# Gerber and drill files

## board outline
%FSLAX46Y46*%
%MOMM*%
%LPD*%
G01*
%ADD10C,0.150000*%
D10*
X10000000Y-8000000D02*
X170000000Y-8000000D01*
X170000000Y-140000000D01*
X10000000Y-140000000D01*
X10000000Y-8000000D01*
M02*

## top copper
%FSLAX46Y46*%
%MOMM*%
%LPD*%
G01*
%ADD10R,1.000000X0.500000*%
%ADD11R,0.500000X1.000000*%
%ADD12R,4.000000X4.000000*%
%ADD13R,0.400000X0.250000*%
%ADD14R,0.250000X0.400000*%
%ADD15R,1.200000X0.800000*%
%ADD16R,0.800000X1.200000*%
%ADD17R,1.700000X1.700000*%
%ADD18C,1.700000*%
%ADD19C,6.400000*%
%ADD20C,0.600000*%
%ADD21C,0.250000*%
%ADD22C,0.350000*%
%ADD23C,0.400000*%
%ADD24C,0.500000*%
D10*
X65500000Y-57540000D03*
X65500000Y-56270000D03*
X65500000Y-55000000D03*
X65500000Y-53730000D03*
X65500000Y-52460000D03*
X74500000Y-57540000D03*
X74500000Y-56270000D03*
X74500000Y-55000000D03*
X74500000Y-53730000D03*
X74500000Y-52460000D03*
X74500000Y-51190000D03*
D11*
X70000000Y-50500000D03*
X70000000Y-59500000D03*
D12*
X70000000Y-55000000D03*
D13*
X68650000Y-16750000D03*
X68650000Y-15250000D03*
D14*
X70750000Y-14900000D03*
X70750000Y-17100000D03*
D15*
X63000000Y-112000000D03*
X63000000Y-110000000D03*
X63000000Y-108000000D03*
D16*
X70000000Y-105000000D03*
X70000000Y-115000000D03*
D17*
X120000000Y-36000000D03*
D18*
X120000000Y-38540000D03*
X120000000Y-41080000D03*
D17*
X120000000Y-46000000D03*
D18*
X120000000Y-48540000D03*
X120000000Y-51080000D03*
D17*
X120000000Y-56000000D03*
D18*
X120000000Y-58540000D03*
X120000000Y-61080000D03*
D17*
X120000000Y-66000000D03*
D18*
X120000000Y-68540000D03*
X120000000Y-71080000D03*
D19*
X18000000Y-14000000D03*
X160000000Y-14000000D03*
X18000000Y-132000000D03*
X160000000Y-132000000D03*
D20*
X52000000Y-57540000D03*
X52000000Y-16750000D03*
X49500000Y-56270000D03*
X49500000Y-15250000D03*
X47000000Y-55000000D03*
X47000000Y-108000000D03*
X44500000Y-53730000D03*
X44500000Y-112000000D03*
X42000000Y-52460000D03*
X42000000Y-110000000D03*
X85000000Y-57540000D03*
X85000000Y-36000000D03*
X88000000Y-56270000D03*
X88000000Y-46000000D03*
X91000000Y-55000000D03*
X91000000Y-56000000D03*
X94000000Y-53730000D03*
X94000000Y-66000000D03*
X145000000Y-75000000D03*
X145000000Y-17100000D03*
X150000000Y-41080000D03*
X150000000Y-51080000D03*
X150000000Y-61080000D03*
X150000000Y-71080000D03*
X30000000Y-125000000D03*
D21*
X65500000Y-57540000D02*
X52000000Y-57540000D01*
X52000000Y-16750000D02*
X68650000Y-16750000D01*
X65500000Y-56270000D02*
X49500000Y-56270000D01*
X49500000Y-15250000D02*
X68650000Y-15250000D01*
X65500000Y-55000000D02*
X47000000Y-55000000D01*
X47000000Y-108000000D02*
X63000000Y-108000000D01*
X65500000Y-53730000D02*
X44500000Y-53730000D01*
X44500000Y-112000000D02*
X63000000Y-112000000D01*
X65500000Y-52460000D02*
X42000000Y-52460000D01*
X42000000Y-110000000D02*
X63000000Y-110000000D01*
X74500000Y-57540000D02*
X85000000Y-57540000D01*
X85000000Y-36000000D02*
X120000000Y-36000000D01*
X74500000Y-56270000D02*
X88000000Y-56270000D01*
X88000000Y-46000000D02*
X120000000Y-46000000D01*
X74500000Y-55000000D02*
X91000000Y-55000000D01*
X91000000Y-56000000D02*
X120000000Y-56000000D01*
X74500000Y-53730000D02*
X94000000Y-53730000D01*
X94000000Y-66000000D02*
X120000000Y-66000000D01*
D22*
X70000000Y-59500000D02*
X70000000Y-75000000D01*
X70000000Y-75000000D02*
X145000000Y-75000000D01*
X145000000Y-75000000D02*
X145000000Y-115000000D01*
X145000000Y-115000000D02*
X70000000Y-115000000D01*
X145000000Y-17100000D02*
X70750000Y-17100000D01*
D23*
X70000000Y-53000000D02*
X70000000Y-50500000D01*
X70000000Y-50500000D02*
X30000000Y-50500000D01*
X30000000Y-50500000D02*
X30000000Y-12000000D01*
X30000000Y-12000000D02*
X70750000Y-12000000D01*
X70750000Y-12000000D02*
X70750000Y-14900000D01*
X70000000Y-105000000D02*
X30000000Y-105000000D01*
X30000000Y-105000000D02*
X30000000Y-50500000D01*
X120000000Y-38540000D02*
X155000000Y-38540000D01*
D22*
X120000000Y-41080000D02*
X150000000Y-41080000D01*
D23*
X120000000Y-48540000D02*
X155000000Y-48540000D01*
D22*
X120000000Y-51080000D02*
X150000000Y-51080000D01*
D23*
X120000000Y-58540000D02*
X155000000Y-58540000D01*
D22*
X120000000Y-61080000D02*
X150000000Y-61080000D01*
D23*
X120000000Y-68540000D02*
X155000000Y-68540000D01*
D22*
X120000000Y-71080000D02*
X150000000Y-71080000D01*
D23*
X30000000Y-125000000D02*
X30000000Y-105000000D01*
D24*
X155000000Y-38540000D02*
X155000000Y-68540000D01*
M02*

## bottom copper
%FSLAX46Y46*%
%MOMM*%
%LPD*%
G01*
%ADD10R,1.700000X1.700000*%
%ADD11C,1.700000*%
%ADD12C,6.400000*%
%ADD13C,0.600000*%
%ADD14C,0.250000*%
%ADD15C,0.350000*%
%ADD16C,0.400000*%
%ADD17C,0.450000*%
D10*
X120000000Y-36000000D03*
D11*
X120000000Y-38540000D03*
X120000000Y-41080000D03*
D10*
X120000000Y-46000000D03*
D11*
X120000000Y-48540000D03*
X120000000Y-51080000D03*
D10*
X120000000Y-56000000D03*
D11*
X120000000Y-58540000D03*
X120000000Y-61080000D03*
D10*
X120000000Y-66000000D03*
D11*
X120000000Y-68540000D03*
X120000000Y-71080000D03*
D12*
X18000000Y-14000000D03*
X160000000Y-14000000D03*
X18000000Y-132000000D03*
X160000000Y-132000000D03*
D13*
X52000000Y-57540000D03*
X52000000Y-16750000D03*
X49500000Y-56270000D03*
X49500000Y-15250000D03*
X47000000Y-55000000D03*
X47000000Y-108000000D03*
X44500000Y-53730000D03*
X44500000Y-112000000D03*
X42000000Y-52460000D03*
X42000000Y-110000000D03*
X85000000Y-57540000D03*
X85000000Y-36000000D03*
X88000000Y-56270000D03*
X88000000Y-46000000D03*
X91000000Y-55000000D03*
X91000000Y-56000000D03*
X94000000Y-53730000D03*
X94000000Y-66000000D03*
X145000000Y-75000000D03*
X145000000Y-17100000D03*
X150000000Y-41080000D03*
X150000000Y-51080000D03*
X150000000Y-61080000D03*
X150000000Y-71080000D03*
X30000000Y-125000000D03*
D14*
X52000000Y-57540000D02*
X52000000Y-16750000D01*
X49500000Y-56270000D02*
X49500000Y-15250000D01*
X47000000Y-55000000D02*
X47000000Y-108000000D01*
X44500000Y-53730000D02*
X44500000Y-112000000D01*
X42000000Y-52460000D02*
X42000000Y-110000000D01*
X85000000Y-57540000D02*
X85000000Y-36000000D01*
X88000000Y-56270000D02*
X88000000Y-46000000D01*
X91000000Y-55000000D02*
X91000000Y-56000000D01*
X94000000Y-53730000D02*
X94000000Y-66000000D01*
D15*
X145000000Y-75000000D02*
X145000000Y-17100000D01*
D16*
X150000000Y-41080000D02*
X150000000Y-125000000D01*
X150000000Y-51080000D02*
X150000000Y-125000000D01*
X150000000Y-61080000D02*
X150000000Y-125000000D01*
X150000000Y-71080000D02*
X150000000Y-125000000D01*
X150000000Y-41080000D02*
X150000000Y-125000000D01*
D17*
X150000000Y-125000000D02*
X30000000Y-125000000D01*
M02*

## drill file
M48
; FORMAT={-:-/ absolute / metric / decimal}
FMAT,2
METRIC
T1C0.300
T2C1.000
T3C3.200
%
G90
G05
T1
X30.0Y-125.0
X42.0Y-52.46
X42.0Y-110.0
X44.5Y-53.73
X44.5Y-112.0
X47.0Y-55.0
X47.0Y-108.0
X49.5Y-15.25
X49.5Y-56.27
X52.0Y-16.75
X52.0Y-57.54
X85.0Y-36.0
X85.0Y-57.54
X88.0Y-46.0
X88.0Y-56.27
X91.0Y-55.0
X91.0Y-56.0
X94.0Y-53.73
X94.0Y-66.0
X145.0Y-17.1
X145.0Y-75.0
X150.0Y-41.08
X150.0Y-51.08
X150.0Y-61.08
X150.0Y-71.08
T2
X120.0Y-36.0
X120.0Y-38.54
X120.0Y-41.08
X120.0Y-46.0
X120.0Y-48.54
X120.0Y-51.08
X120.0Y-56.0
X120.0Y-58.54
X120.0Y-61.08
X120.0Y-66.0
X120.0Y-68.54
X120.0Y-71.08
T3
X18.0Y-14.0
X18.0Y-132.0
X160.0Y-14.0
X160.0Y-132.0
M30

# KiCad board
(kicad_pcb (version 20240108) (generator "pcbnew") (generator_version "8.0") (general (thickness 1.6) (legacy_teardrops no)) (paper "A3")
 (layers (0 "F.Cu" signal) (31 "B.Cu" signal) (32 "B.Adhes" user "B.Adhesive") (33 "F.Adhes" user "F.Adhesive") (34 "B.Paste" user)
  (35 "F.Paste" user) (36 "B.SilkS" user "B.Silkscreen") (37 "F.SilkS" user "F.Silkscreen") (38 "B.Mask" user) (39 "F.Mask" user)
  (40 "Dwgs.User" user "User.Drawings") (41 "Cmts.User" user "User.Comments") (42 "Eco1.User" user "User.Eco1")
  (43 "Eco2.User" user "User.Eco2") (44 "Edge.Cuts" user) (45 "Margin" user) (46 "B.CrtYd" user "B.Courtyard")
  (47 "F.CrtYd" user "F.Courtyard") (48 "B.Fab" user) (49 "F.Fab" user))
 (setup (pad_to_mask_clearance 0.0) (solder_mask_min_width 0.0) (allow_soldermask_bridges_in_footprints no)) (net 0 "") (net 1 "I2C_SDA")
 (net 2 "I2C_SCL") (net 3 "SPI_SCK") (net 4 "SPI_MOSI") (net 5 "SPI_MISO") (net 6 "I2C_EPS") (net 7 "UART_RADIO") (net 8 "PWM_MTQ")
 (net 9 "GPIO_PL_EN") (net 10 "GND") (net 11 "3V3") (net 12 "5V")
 (gr_rect (start 10 8) (end 170 140) (stroke (width 0.15) (type solid)) (fill none) (layer "Edge.Cuts"))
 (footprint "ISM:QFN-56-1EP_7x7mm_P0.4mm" (layer "F.Cu") (at 70 55)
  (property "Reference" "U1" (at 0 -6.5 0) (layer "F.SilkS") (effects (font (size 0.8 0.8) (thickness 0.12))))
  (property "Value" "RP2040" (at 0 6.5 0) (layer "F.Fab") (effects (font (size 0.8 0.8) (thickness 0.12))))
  (pad "1" smd rect (at -4.5 2.54) (size 1.0 0.5) (layers "F.Cu" "F.Paste" "F.Mask") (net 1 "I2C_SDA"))
  (pad "2" smd rect (at -4.5 1.27) (size 1.0 0.5) (layers "F.Cu" "F.Paste" "F.Mask") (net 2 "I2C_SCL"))
  (pad "3" smd rect (at -4.5 0) (size 1.0 0.5) (layers "F.Cu" "F.Paste" "F.Mask") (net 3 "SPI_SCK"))
  (pad "4" smd rect (at -4.5 -1.27) (size 1.0 0.5) (layers "F.Cu" "F.Paste" "F.Mask") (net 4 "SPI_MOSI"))
  (pad "5" smd rect (at -4.5 -2.54) (size 1.0 0.5) (layers "F.Cu" "F.Paste" "F.Mask") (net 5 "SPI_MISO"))
  (pad "6" smd rect (at 4.5 2.54) (size 1.0 0.5) (layers "F.Cu" "F.Paste" "F.Mask") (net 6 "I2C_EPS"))
  (pad "7" smd rect (at 4.5 1.27) (size 1.0 0.5) (layers "F.Cu" "F.Paste" "F.Mask") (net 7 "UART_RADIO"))
  (pad "8" smd rect (at 4.5 0) (size 1.0 0.5) (layers "F.Cu" "F.Paste" "F.Mask") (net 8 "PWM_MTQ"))
  (pad "9" smd rect (at 4.5 -1.27) (size 1.0 0.5) (layers "F.Cu" "F.Paste" "F.Mask") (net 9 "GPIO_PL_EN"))
  (pad "12" smd rect (at 4.5 -2.54) (size 1.0 0.5) (layers "F.Cu" "F.Paste" "F.Mask"))
  (pad "13" smd rect (at 4.5 -3.81) (size 1.0 0.5) (layers "F.Cu" "F.Paste" "F.Mask"))
  (pad "10" smd rect (at 0 -4.5) (size 0.5 1.0) (layers "F.Cu" "F.Paste" "F.Mask") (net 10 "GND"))
  (pad "11" smd rect (at 0 4.5) (size 0.5 1.0) (layers "F.Cu" "F.Paste" "F.Mask") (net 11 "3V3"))
  (pad "EP" smd rect (at 0 0) (size 4 4) (layers "F.Cu" "F.Paste" "F.Mask") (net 10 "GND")))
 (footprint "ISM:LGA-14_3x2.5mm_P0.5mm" (layer "F.Cu") (at 70 16)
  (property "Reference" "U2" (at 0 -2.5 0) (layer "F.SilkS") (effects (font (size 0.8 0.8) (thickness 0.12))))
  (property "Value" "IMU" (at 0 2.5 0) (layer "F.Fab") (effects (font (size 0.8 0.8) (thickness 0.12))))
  (pad "1" smd rect (at -1.35 0.75) (size 0.4 0.25) (layers "F.Cu" "F.Paste" "F.Mask") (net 1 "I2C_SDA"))
  (pad "2" smd rect (at -1.35 -0.75) (size 0.4 0.25) (layers "F.Cu" "F.Paste" "F.Mask") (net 2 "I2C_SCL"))
  (pad "3" smd rect (at 0.75 -1.1) (size 0.25 0.4) (layers "F.Cu" "F.Paste" "F.Mask") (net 10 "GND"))
  (pad "4" smd rect (at 0.75 1.1) (size 0.25 0.4) (layers "F.Cu" "F.Paste" "F.Mask") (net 11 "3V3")))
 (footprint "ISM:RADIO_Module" (layer "F.Cu") (at 70 110)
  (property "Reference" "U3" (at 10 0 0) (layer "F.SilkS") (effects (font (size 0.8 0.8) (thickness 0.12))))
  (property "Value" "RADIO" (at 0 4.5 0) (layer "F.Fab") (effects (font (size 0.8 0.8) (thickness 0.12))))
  (pad "1" smd rect (at -7 2) (size 1.2 0.8) (layers "F.Cu" "F.Paste" "F.Mask") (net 4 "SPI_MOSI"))
  (pad "2" smd rect (at -7 0) (size 1.2 0.8) (layers "F.Cu" "F.Paste" "F.Mask") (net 5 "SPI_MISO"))
  (pad "3" smd rect (at -7 -2) (size 1.2 0.8) (layers "F.Cu" "F.Paste" "F.Mask") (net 3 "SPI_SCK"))
  (pad "4" smd rect (at 0 -5) (size 0.8 1.2) (layers "F.Cu" "F.Paste" "F.Mask") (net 10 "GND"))
  (pad "5" smd rect (at 0 5) (size 0.8 1.2) (layers "F.Cu" "F.Paste" "F.Mask") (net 11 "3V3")))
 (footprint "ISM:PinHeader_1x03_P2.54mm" (layer "F.Cu") (at 120 36)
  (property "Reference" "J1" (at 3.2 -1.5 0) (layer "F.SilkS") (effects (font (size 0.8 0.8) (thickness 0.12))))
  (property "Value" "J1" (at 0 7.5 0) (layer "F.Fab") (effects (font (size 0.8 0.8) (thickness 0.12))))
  (pad "1" thru_hole rect (at 0 0) (size 1.7 1.7) (drill 1.0) (layers "*.Cu" "*.Mask") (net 6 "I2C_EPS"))
  (pad "2" thru_hole circle (at 0 2.54) (size 1.7 1.7) (drill 1.0) (layers "*.Cu" "*.Mask") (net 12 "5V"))
  (pad "3" thru_hole circle (at 0 5.08) (size 1.7 1.7) (drill 1.0) (layers "*.Cu" "*.Mask") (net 10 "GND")))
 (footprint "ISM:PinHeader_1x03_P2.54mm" (layer "F.Cu") (at 120 46)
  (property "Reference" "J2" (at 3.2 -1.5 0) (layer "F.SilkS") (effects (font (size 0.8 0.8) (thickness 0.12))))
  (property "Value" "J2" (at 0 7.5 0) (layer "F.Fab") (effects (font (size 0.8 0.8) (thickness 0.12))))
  (pad "1" thru_hole rect (at 0 0) (size 1.7 1.7) (drill 1.0) (layers "*.Cu" "*.Mask") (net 7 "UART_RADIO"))
  (pad "2" thru_hole circle (at 0 2.54) (size 1.7 1.7) (drill 1.0) (layers "*.Cu" "*.Mask") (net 12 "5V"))
  (pad "3" thru_hole circle (at 0 5.08) (size 1.7 1.7) (drill 1.0) (layers "*.Cu" "*.Mask") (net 10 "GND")))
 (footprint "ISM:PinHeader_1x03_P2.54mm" (layer "F.Cu") (at 120 56)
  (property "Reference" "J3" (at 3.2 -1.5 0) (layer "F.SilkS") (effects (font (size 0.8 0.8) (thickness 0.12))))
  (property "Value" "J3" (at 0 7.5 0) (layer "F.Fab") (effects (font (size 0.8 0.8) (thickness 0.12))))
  (pad "1" thru_hole rect (at 0 0) (size 1.7 1.7) (drill 1.0) (layers "*.Cu" "*.Mask") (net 8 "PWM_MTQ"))
  (pad "2" thru_hole circle (at 0 2.54) (size 1.7 1.7) (drill 1.0) (layers "*.Cu" "*.Mask") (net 12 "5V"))
  (pad "3" thru_hole circle (at 0 5.08) (size 1.7 1.7) (drill 1.0) (layers "*.Cu" "*.Mask") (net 10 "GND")))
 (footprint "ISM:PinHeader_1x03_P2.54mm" (layer "F.Cu") (at 120 66)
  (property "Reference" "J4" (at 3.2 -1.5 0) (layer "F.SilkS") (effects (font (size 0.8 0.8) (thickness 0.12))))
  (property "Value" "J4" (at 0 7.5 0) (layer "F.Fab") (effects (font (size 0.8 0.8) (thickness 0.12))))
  (pad "1" thru_hole rect (at 0 0) (size 1.7 1.7) (drill 1.0) (layers "*.Cu" "*.Mask") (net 9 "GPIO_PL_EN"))
  (pad "2" thru_hole circle (at 0 2.54) (size 1.7 1.7) (drill 1.0) (layers "*.Cu" "*.Mask") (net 12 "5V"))
  (pad "3" thru_hole circle (at 0 5.08) (size 1.7 1.7) (drill 1.0) (layers "*.Cu" "*.Mask") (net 10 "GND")))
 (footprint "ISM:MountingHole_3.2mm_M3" (layer "F.Cu") (at 18 14)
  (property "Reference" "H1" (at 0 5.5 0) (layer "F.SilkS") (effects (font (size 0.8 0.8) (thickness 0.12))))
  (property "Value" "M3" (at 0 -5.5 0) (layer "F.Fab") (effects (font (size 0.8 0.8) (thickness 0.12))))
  (pad "" thru_hole circle (at 0 0) (size 6.4 6.4) (drill 3.2) (layers "*.Cu" "*.Mask")))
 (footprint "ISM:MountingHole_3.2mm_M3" (layer "F.Cu") (at 160 14)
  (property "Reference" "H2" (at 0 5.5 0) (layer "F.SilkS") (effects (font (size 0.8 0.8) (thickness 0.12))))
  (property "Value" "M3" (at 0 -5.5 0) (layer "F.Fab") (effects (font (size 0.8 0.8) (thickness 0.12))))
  (pad "" thru_hole circle (at 0 0) (size 6.4 6.4) (drill 3.2) (layers "*.Cu" "*.Mask")))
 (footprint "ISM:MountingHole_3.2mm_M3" (layer "F.Cu") (at 18 132)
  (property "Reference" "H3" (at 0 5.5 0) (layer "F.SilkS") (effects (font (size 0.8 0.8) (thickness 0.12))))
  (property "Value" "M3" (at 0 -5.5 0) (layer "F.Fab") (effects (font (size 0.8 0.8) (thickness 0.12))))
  (pad "" thru_hole circle (at 0 0) (size 6.4 6.4) (drill 3.2) (layers "*.Cu" "*.Mask")))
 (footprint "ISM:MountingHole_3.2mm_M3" (layer "F.Cu") (at 160 132)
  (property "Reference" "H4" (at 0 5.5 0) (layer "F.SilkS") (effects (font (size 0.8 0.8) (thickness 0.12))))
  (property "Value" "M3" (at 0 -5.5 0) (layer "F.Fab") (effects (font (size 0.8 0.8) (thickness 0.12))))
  (pad "" thru_hole circle (at 0 0) (size 6.4 6.4) (drill 3.2) (layers "*.Cu" "*.Mask")))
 (segment (start 65.5 57.54) (end 52.0 57.54) (width 0.25) (layer "F.Cu") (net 1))
 (segment (start 52.0 57.54) (end 52.0 16.75) (width 0.25) (layer "B.Cu") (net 1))
 (segment (start 52.0 16.75) (end 68.65 16.75) (width 0.25) (layer "F.Cu") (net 1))
 (segment (start 65.5 56.27) (end 49.5 56.27) (width 0.25) (layer "F.Cu") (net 2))
 (segment (start 49.5 56.27) (end 49.5 15.25) (width 0.25) (layer "B.Cu") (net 2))
 (segment (start 49.5 15.25) (end 68.65 15.25) (width 0.25) (layer "F.Cu") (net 2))
 (segment (start 65.5 55) (end 47.0 55) (width 0.25) (layer "F.Cu") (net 3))
 (segment (start 47.0 55) (end 47.0 108) (width 0.25) (layer "B.Cu") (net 3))
 (segment (start 47.0 108) (end 63 108) (width 0.25) (layer "F.Cu") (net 3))
 (segment (start 65.5 53.73) (end 44.5 53.73) (width 0.25) (layer "F.Cu") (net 4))
 (segment (start 44.5 53.73) (end 44.5 112) (width 0.25) (layer "B.Cu") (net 4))
 (segment (start 44.5 112) (end 63 112) (width 0.25) (layer "F.Cu") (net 4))
 (segment (start 65.5 52.46) (end 42.0 52.46) (width 0.25) (layer "F.Cu") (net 5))
 (segment (start 42.0 52.46) (end 42.0 110) (width 0.25) (layer "B.Cu") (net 5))
 (segment (start 42.0 110) (end 63 110) (width 0.25) (layer "F.Cu") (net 5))
 (segment (start 74.5 57.54) (end 85 57.54) (width 0.25) (layer "F.Cu") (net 6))
 (segment (start 85 57.54) (end 85 36) (width 0.25) (layer "B.Cu") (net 6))
 (segment (start 85 36) (end 120 36) (width 0.25) (layer "F.Cu") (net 6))
 (segment (start 74.5 56.27) (end 88 56.27) (width 0.25) (layer "F.Cu") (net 7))
 (segment (start 88 56.27) (end 88 46) (width 0.25) (layer "B.Cu") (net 7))
 (segment (start 88 46) (end 120 46) (width 0.25) (layer "F.Cu") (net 7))
 (segment (start 74.5 55) (end 91 55) (width 0.25) (layer "F.Cu") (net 8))
 (segment (start 91 55) (end 91 56) (width 0.25) (layer "B.Cu") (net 8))
 (segment (start 91 56) (end 120 56) (width 0.25) (layer "F.Cu") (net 8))
 (segment (start 74.5 53.73) (end 94 53.73) (width 0.25) (layer "F.Cu") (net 9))
 (segment (start 94 53.73) (end 94 66) (width 0.25) (layer "B.Cu") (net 9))
 (segment (start 94 66) (end 120 66) (width 0.25) (layer "F.Cu") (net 9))
 (segment (start 70 59.5) (end 70 75) (width 0.35) (layer "F.Cu") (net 11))
 (segment (start 70 75) (end 145 75) (width 0.35) (layer "F.Cu") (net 11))
 (segment (start 145 75) (end 145 115) (width 0.35) (layer "F.Cu") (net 11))
 (segment (start 145 115) (end 70 115) (width 0.35) (layer "F.Cu") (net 11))
 (segment (start 145 75) (end 145 17.1) (width 0.35) (layer "B.Cu") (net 11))
 (segment (start 145 17.1) (end 70.75 17.1) (width 0.35) (layer "F.Cu") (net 11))
 (segment (start 70 53) (end 70 50.5) (width 0.4) (layer "F.Cu") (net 10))
 (segment (start 70 50.5) (end 30 50.5) (width 0.4) (layer "F.Cu") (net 10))
 (segment (start 30 50.5) (end 30 12) (width 0.4) (layer "F.Cu") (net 10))
 (segment (start 30 12) (end 70.75 12) (width 0.4) (layer "F.Cu") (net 10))
 (segment (start 70.75 12) (end 70.75 14.9) (width 0.4) (layer "F.Cu") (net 10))
 (segment (start 70 105) (end 30 105) (width 0.4) (layer "F.Cu") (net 10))
 (segment (start 30 105) (end 30 50.5) (width 0.4) (layer "F.Cu") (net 10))
 (segment (start 120 38.54) (end 155 38.54) (width 0.4) (layer "F.Cu") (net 12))
 (segment (start 120 41.08) (end 150 41.08) (width 0.35) (layer "F.Cu") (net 10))
 (segment (start 150 41.08) (end 150 125) (width 0.4) (layer "B.Cu") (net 10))
 (segment (start 120 48.54) (end 155 48.54) (width 0.4) (layer "F.Cu") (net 12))
 (segment (start 120 51.08) (end 150 51.08) (width 0.35) (layer "F.Cu") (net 10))
 (segment (start 150 51.08) (end 150 125) (width 0.4) (layer "B.Cu") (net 10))
 (segment (start 120 58.54) (end 155 58.54) (width 0.4) (layer "F.Cu") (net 12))
 (segment (start 120 61.08) (end 150 61.08) (width 0.35) (layer "F.Cu") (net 10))
 (segment (start 150 61.08) (end 150 125) (width 0.4) (layer "B.Cu") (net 10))
 (segment (start 120 68.54) (end 155 68.54) (width 0.4) (layer "F.Cu") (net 12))
 (segment (start 120 71.08) (end 150 71.08) (width 0.35) (layer "F.Cu") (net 10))
 (segment (start 150 71.08) (end 150 125) (width 0.4) (layer "B.Cu") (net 10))
 (segment (start 150 41.08) (end 150 125) (width 0.4) (layer "B.Cu") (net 10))
 (segment (start 150 125) (end 30 125) (width 0.45) (layer "B.Cu") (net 10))
 (segment (start 30 125) (end 30 105) (width 0.4) (layer "F.Cu") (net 10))
 (segment (start 155 38.54) (end 155 68.54) (width 0.5) (layer "F.Cu") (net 12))
 (via (at 52.0 57.54) (size 0.6) (drill 0.3) (layers "F.Cu" "B.Cu") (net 1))
 (via (at 52.0 16.75) (size 0.6) (drill 0.3) (layers "F.Cu" "B.Cu") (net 1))
 (via (at 49.5 56.27) (size 0.6) (drill 0.3) (layers "F.Cu" "B.Cu") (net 2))
 (via (at 49.5 15.25) (size 0.6) (drill 0.3) (layers "F.Cu" "B.Cu") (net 2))
 (via (at 47.0 55) (size 0.6) (drill 0.3) (layers "F.Cu" "B.Cu") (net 3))
 (via (at 47.0 108) (size 0.6) (drill 0.3) (layers "F.Cu" "B.Cu") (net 3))
 (via (at 44.5 53.73) (size 0.6) (drill 0.3) (layers "F.Cu" "B.Cu") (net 4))
 (via (at 44.5 112) (size 0.6) (drill 0.3) (layers "F.Cu" "B.Cu") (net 4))
 (via (at 42.0 52.46) (size 0.6) (drill 0.3) (layers "F.Cu" "B.Cu") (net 5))
 (via (at 42.0 110) (size 0.6) (drill 0.3) (layers "F.Cu" "B.Cu") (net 5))
 (via (at 85 57.54) (size 0.6) (drill 0.3) (layers "F.Cu" "B.Cu") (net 6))
 (via (at 85 36) (size 0.6) (drill 0.3) (layers "F.Cu" "B.Cu") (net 6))
 (via (at 88 56.27) (size 0.6) (drill 0.3) (layers "F.Cu" "B.Cu") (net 7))
 (via (at 88 46) (size 0.6) (drill 0.3) (layers "F.Cu" "B.Cu") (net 7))
 (via (at 91 55) (size 0.6) (drill 0.3) (layers "F.Cu" "B.Cu") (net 8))
 (via (at 91 56) (size 0.6) (drill 0.3) (layers "F.Cu" "B.Cu") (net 8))
 (via (at 94 53.73) (size 0.6) (drill 0.3) (layers "F.Cu" "B.Cu") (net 9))
 (via (at 94 66) (size 0.6) (drill 0.3) (layers "F.Cu" "B.Cu") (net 9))
 (via (at 145 75) (size 0.6) (drill 0.3) (layers "F.Cu" "B.Cu") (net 11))
 (via (at 145 17.1) (size 0.6) (drill 0.3) (layers "F.Cu" "B.Cu") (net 11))
 (via (at 150 41.08) (size 0.6) (drill 0.3) (layers "F.Cu" "B.Cu") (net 10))
 (via (at 150 51.08) (size 0.6) (drill 0.3) (layers "F.Cu" "B.Cu") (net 10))
 (via (at 150 61.08) (size 0.6) (drill 0.3) (layers "F.Cu" "B.Cu") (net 10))
 (via (at 150 71.08) (size 0.6) (drill 0.3) (layers "F.Cu" "B.Cu") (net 10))
 (via (at 30 125) (size 0.6) (drill 0.3) (layers "F.Cu" "B.Cu") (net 10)))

